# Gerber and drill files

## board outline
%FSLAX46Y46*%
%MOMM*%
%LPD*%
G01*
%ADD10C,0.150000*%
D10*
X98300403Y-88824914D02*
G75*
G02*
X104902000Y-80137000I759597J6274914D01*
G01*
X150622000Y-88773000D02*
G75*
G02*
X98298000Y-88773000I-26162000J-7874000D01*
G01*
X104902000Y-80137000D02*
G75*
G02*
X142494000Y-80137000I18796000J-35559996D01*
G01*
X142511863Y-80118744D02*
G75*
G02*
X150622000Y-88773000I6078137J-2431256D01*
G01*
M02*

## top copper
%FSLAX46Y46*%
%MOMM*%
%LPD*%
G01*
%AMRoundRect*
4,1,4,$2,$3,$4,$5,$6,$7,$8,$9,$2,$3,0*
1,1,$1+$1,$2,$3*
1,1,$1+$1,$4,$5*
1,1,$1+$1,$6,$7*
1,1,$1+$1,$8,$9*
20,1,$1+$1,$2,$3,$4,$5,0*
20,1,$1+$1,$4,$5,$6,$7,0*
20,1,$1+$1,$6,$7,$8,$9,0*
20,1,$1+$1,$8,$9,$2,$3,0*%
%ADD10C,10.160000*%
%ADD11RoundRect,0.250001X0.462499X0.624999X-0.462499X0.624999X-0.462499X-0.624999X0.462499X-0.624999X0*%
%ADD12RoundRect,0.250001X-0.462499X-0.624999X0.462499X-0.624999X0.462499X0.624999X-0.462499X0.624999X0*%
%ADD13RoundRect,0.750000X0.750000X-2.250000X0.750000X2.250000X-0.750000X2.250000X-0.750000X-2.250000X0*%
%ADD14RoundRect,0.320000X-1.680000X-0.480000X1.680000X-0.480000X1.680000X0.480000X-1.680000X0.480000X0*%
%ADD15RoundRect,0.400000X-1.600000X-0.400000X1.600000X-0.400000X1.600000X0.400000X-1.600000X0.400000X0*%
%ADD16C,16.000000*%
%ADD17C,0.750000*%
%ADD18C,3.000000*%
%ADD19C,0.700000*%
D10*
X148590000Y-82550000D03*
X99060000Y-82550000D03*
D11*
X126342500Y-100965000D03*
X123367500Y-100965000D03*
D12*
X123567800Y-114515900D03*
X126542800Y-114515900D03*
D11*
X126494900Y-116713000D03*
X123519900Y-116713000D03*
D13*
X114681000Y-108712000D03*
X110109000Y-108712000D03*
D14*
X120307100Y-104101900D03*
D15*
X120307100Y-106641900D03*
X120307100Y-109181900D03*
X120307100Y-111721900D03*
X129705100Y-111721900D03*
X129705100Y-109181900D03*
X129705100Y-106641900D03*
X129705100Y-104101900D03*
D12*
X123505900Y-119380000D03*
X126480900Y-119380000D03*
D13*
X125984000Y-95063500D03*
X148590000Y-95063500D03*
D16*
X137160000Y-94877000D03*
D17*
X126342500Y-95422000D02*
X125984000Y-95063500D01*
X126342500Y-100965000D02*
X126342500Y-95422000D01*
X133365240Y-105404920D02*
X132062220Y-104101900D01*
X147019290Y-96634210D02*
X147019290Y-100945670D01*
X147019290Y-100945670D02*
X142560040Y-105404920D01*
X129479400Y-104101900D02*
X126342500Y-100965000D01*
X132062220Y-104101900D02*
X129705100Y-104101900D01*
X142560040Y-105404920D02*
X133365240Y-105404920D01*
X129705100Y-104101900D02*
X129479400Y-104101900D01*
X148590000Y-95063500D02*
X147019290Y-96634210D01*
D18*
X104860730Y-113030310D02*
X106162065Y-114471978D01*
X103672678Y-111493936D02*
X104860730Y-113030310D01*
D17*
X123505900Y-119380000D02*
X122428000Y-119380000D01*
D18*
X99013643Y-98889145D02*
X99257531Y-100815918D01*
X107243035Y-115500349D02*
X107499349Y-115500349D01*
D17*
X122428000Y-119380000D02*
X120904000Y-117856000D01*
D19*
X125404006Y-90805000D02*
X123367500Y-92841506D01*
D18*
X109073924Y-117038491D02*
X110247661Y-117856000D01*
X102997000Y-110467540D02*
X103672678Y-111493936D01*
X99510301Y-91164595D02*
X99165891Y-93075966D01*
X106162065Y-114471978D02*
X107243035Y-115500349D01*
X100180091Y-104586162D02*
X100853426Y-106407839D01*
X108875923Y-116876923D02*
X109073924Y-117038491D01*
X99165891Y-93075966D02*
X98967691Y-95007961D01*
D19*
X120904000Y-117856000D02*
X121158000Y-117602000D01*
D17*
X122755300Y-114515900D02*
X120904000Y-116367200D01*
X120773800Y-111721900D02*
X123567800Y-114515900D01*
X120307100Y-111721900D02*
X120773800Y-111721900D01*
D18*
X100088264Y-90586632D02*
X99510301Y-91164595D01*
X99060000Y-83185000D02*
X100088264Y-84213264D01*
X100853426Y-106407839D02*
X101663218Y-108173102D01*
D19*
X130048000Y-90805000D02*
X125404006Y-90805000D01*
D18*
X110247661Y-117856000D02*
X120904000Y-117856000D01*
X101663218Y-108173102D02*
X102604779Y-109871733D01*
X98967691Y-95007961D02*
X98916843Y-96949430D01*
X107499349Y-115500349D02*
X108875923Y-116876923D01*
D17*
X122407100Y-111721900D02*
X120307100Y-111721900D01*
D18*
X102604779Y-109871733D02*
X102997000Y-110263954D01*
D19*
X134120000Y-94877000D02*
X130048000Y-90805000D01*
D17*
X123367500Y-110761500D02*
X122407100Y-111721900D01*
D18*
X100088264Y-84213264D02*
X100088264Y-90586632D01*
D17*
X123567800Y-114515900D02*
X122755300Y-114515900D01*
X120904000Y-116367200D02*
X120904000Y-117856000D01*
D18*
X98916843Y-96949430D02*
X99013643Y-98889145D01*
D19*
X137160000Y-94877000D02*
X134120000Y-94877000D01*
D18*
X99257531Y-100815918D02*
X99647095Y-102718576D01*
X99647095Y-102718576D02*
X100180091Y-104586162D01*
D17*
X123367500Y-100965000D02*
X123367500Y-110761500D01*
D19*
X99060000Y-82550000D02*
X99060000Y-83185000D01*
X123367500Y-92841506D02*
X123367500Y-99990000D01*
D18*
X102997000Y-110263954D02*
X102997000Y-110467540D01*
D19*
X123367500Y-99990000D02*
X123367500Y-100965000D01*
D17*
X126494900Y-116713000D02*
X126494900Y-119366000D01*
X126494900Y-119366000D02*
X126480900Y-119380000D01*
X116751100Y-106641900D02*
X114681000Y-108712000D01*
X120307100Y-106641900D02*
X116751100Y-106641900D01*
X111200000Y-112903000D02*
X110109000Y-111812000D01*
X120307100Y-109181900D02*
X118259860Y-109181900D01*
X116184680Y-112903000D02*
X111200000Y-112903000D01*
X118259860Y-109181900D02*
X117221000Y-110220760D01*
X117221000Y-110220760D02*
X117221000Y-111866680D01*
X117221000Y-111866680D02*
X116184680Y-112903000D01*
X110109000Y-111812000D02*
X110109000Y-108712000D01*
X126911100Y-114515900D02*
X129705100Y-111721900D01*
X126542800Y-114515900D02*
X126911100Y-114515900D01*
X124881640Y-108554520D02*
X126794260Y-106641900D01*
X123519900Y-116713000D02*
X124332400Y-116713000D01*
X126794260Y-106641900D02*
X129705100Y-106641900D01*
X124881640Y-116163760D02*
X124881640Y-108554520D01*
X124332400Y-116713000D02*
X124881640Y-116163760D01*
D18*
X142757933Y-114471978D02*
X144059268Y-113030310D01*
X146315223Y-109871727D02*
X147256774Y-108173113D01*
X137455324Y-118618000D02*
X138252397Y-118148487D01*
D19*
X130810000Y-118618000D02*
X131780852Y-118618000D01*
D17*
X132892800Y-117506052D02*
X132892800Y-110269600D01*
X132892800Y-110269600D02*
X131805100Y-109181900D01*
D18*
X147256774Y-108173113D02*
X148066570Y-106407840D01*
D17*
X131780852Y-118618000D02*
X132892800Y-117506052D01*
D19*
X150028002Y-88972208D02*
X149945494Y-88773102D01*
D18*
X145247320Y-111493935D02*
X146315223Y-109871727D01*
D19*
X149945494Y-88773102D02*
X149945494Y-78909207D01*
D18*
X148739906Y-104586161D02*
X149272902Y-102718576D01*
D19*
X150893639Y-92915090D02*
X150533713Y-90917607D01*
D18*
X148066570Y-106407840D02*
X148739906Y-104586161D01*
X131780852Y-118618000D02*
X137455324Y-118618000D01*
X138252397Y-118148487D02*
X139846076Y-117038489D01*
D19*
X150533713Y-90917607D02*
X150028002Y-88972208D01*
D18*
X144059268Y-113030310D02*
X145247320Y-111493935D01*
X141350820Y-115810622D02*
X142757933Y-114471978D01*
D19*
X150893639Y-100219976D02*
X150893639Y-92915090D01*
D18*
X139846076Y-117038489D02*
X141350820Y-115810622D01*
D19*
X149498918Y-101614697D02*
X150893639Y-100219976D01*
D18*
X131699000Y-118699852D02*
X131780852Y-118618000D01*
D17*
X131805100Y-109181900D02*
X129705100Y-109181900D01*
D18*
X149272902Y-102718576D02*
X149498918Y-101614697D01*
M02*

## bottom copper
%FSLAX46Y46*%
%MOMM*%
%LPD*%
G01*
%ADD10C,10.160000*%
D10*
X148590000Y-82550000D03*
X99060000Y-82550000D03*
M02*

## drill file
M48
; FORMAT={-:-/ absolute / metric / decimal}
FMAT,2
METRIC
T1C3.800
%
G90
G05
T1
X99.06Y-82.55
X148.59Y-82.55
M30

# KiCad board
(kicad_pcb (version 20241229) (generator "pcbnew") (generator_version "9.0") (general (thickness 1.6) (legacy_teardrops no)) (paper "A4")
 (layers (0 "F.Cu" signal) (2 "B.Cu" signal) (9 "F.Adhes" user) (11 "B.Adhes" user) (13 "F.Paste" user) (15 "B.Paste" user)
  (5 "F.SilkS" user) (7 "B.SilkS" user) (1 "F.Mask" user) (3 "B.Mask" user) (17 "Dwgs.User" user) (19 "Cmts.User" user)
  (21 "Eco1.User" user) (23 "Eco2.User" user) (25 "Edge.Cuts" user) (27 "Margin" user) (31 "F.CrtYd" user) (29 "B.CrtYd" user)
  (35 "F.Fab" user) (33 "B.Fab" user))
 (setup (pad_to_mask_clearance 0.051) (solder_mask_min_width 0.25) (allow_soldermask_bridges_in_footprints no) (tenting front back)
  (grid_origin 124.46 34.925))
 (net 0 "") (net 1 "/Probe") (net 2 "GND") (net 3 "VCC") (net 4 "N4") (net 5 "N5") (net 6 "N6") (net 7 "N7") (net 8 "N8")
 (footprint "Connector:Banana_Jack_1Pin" (layer "F.Cu") (at 148.59 82.55)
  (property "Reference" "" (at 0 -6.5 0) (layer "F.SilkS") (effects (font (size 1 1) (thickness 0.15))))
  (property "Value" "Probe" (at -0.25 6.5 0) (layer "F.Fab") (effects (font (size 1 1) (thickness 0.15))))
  (pad "1" thru_hole circle (at 0 0) (size 10.16 10.16) (drill 3.8) (layers "*.Cu" "*.Mask") (remove_unused_layers no) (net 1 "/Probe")))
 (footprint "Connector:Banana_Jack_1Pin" (layer "F.Cu") (at 99.06 82.55)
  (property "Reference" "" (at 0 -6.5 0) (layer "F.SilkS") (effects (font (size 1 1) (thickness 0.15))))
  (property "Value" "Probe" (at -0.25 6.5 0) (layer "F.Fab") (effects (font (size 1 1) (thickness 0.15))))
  (pad "1" thru_hole circle (at 0 0) (size 10.16 10.16) (drill 3.8) (layers "*.Cu" "*.Mask") (remove_unused_layers no) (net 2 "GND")))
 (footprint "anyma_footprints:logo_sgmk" (layer "F.Cu") (at 135.382 110.744)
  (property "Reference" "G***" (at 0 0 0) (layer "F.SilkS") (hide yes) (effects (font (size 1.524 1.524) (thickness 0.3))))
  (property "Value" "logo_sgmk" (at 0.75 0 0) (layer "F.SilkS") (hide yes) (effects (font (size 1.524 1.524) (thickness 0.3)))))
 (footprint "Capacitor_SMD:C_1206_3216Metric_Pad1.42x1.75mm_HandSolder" (layer "F.Cu") (at 124.855 100.965 180)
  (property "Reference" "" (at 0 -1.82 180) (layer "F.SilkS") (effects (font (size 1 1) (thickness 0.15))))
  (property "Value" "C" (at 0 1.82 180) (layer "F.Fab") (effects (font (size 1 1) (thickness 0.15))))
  (pad "1" smd roundrect (at -1.4875 0 180) (size 1.425 1.75) (layers "F.Cu" "F.Mask" "F.Paste") (roundrect_rratio 0.175439) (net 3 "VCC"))
  (pad "2" smd roundrect (at 1.4875 0 180) (size 1.425 1.75) (layers "F.Cu" "F.Mask" "F.Paste") (roundrect_rratio 0.175439) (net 2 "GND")))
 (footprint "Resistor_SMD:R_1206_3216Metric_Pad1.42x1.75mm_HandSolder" (layer "F.Cu") (at 125.0553 114.5159)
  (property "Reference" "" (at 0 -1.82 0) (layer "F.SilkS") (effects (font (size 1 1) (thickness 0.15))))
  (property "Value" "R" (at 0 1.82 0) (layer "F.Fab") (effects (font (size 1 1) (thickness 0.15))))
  (pad "1" smd roundrect (at -1.4875 0) (size 1.425 1.75) (layers "F.Cu" "F.Mask" "F.Paste") (roundrect_rratio 0.175439) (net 2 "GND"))
  (pad "2" smd roundrect (at 1.4875 0) (size 1.425 1.75) (layers "F.Cu" "F.Mask" "F.Paste") (roundrect_rratio 0.175439) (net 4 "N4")))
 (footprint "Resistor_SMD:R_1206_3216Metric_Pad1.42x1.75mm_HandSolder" (layer "F.Cu") (at 125.0074 116.713 180)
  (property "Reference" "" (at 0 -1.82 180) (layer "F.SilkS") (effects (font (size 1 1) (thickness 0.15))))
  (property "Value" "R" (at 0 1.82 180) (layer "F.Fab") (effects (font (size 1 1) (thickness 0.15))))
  (pad "1" smd roundrect (at -1.4875 0 180) (size 1.425 1.75) (layers "F.Cu" "F.Mask" "F.Paste") (roundrect_rratio 0.175439) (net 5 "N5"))
  (pad "2" smd roundrect (at 1.4875 0 180) (size 1.425 1.75) (layers "F.Cu" "F.Mask" "F.Paste") (roundrect_rratio 0.175439) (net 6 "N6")))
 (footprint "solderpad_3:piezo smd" (layer "F.Cu") (at 112.395 93.98 -90)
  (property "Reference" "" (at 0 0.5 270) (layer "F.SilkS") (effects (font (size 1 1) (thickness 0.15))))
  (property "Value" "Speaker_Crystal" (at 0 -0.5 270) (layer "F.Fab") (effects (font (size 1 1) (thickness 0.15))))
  (pad "1" smd roundrect (at 14.732 -2.286 90) (size 6 3) (layers "F.Cu" "F.Mask" "F.Paste") (roundrect_rratio 0.25) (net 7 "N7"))
  (pad "2" smd roundrect (at 14.732 2.286 90) (size 6 3) (layers "F.Cu" "F.Mask" "F.Paste") (roundrect_rratio 0.25) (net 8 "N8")))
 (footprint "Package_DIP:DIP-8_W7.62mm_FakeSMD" (layer "F.Cu") (at 121.1961 104.1019)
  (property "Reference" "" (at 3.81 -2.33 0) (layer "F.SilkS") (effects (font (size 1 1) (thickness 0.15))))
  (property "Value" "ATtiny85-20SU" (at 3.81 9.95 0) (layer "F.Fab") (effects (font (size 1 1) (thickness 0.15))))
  (pad "1" smd roundrect (at -0.889 0) (size 4 1.6) (layers "F.Cu" "F.Mask" "F.Paste") (roundrect_rratio 0.2))
  (pad "2" smd roundrect (at -0.889 2.54) (size 4 1.6) (layers "F.Cu" "F.Mask" "F.Paste") (roundrect_rratio 0.25) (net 7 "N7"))
  (pad "3" smd roundrect (at -0.889 5.08) (size 4 1.6) (layers "F.Cu" "F.Mask" "F.Paste") (roundrect_rratio 0.25) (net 8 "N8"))
  (pad "4" smd roundrect (at -0.889 7.62) (size 4 1.6) (layers "F.Cu" "F.Mask" "F.Paste") (roundrect_rratio 0.25) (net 2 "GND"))
  (pad "5" smd roundrect (at 8.509 7.62) (size 4 1.6) (layers "F.Cu" "F.Mask" "F.Paste") (roundrect_rratio 0.25) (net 4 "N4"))
  (pad "6" smd roundrect (at 8.509 5.08) (size 4 1.6) (layers "F.Cu" "F.Mask" "F.Paste") (roundrect_rratio 0.25) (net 1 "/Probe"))
  (pad "7" smd roundrect (at 8.509 2.54) (size 4 1.6) (layers "F.Cu" "F.Mask" "F.Paste") (roundrect_rratio 0.25) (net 6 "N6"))
  (pad "8" smd roundrect (at 8.509 0) (size 4 1.6) (layers "F.Cu" "F.Mask" "F.Paste") (roundrect_rratio 0.25) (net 3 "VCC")))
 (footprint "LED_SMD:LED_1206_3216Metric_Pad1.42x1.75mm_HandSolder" (layer "F.Cu") (at 124.9934 119.38)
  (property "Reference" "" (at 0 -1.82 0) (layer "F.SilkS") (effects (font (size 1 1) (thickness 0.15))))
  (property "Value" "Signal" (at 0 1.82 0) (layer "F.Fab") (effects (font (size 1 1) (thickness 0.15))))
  (pad "1" smd roundrect (at -1.4875 0) (size 1.425 1.75) (layers "F.Cu" "F.Mask" "F.Paste") (roundrect_rratio 0.175439) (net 2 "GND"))
  (pad "2" smd roundrect (at 1.4875 0) (size 1.425 1.75) (layers "F.Cu" "F.Mask" "F.Paste") (roundrect_rratio 0.175439) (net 5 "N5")))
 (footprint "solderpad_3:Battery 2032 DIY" (layer "F.Cu") (at 137.16 95.0635)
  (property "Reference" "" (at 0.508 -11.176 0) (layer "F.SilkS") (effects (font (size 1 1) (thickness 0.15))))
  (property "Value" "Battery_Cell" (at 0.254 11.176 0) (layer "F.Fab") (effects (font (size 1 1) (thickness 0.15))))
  (pad "1" smd roundrect (at -11.176 0 90) (size 6 3) (layers "F.Cu" "F.Mask" "F.Paste") (roundrect_rratio 0.25) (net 3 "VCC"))
  (pad "1" smd roundrect (at 11.43 0 90) (size 6 3) (layers "F.Cu" "F.Mask" "F.Paste") (roundrect_rratio 0.25) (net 3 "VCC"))
  (pad "2" smd circle (at 0 -0.1865) (size 16 16) (layers "F.Cu" "F.Mask" "F.Paste") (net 2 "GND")))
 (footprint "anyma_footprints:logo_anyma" (layer "B.Cu") (at 125.222 99.441 180)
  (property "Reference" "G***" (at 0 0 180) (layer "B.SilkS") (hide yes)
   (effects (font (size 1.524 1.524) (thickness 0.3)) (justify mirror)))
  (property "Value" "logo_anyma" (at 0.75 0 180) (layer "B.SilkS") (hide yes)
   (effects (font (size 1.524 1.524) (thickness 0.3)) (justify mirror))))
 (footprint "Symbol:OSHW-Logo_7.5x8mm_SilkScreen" (layer "B.Cu") (at 125.349 111.506 180)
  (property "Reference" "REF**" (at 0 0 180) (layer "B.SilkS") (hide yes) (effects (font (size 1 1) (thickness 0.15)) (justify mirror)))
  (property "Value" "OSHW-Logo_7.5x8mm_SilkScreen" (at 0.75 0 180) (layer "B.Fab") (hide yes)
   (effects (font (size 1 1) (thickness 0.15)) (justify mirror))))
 (gr_arc (start 98.300403 88.824914) (mid 94.02734 78.725884) (end 104.902 80.137) (stroke (width 0.15) (type solid)) (layer "Edge.Cuts"))
 (gr_arc (start 150.622 88.773) (mid 124.46 123.968239) (end 98.298 88.773) (stroke (width 0.15) (type solid)) (layer "Edge.Cuts"))
 (gr_arc (start 104.902 80.137) (mid 123.698 75.475075) (end 142.494 80.137) (stroke (width 0.15) (type solid)) (layer "Edge.Cuts"))
 (gr_arc (start 142.511863 80.118744) (mid 153.366698 78.073627) (end 150.622 88.773) (stroke (width 0.15) (type solid)) (layer "Edge.Cuts"))
 (segment (start 126.3425 95.422) (end 125.984 95.0635) (width 0.75) (layer "F.Cu") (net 3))
 (segment (start 126.3425 100.965) (end 126.3425 95.422) (width 0.75) (layer "F.Cu") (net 3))
 (segment (start 133.36524 105.40492) (end 132.06222 104.1019) (width 0.75) (layer "F.Cu") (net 3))
 (segment (start 147.01929 96.63421) (end 147.01929 100.94567) (width 0.75) (layer "F.Cu") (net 3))
 (segment (start 147.01929 100.94567) (end 142.56004 105.40492) (width 0.75) (layer "F.Cu") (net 3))
 (segment (start 129.4794 104.1019) (end 126.3425 100.965) (width 0.75) (layer "F.Cu") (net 3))
 (segment (start 132.06222 104.1019) (end 129.7051 104.1019) (width 0.75) (layer "F.Cu") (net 3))
 (segment (start 142.56004 105.40492) (end 133.36524 105.40492) (width 0.75) (layer "F.Cu") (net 3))
 (segment (start 129.7051 104.1019) (end 129.4794 104.1019) (width 0.75) (layer "F.Cu") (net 3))
 (segment (start 148.59 95.0635) (end 147.01929 96.63421) (width 0.75) (layer "F.Cu") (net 3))
 (segment (start 104.86073 113.03031) (end 106.162065 114.471978) (width 3) (layer "F.Cu") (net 2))
 (segment (start 103.672678 111.493936) (end 104.86073 113.03031) (width 3) (layer "F.Cu") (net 2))
 (segment (start 123.5059 119.38) (end 122.428 119.38) (width 0.75) (layer "F.Cu") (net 2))
 (segment (start 99.013643 98.889145) (end 99.257531 100.815918) (width 3) (layer "F.Cu") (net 2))
 (segment (start 107.243035 115.500349) (end 107.499349 115.500349) (width 3) (layer "F.Cu") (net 2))
 (segment (start 122.428 119.38) (end 120.904 117.856) (width 0.75) (layer "F.Cu") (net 2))
 (segment (start 125.404006 90.805) (end 123.3675 92.841506) (width 0.7) (layer "F.Cu") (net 2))
 (segment (start 109.073924 117.038491) (end 110.247661 117.856) (width 3) (layer "F.Cu") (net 2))
 (segment (start 102.997 110.46754) (end 103.672678 111.493936) (width 3) (layer "F.Cu") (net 2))
 (segment (start 99.510301 91.164595) (end 99.165891 93.075966) (width 3) (layer "F.Cu") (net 2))
 (segment (start 106.162065 114.471978) (end 107.243035 115.500349) (width 3) (layer "F.Cu") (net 2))
 (segment (start 100.180091 104.586162) (end 100.853426 106.407839) (width 3) (layer "F.Cu") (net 2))
 (segment (start 108.875923 116.876923) (end 109.073924 117.038491) (width 3) (layer "F.Cu") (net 2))
 (segment (start 99.165891 93.075966) (end 98.967691 95.007961) (width 3) (layer "F.Cu") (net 2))
 (segment (start 120.904 117.856) (end 121.158 117.602) (width 0.7) (layer "F.Cu") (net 2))
 (segment (start 122.7553 114.5159) (end 120.904 116.3672) (width 0.75) (layer "F.Cu") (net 2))
 (segment (start 120.7738 111.7219) (end 123.5678 114.5159) (width 0.75) (layer "F.Cu") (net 2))
 (segment (start 120.3071 111.7219) (end 120.7738 111.7219) (width 0.75) (layer "F.Cu") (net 2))
 (segment (start 100.088264 90.586632) (end 99.510301 91.164595) (width 3) (layer "F.Cu") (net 2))
 (segment (start 99.06 83.185) (end 100.088264 84.213264) (width 3) (layer "F.Cu") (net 2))
 (segment (start 100.853426 106.407839) (end 101.663218 108.173102) (width 3) (layer "F.Cu") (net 2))
 (segment (start 130.048 90.805) (end 125.404006 90.805) (width 0.7) (layer "F.Cu") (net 2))
 (segment (start 110.247661 117.856) (end 120.904 117.856) (width 3) (layer "F.Cu") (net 2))
 (segment (start 101.663218 108.173102) (end 102.604779 109.871733) (width 3) (layer "F.Cu") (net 2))
 (segment (start 98.967691 95.007961) (end 98.916843 96.94943) (width 3) (layer "F.Cu") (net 2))
 (segment (start 107.499349 115.500349) (end 108.875923 116.876923) (width 3) (layer "F.Cu") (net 2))
 (segment (start 122.4071 111.7219) (end 120.3071 111.7219) (width 0.75) (layer "F.Cu") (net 2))
 (segment (start 102.604779 109.871733) (end 102.997 110.263954) (width 3) (layer "F.Cu") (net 2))
 (segment (start 134.12 94.877) (end 130.048 90.805) (width 0.7) (layer "F.Cu") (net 2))
 (segment (start 123.3675 110.7615) (end 122.4071 111.7219) (width 0.75) (layer "F.Cu") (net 2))
 (segment (start 100.088264 84.213264) (end 100.088264 90.586632) (width 3) (layer "F.Cu") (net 2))
 (segment (start 123.5678 114.5159) (end 122.7553 114.5159) (width 0.75) (layer "F.Cu") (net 2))
 (segment (start 120.904 116.3672) (end 120.904 117.856) (width 0.75) (layer "F.Cu") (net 2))
 (segment (start 98.916843 96.94943) (end 99.013643 98.889145) (width 3) (layer "F.Cu") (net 2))
 (segment (start 137.16 94.877) (end 134.12 94.877) (width 0.7) (layer "F.Cu") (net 2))
 (segment (start 99.257531 100.815918) (end 99.647095 102.718576) (width 3) (layer "F.Cu") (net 2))
 (segment (start 99.647095 102.718576) (end 100.180091 104.586162) (width 3) (layer "F.Cu") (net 2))
 (segment (start 123.3675 100.965) (end 123.3675 110.7615) (width 0.75) (layer "F.Cu") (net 2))
 (segment (start 99.06 82.55) (end 99.06 83.185) (width 0.7) (layer "F.Cu") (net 2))
 (segment (start 123.3675 92.841506) (end 123.3675 99.99) (width 0.7) (layer "F.Cu") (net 2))
 (segment (start 102.997 110.263954) (end 102.997 110.46754) (width 3) (layer "F.Cu") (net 2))
 (segment (start 123.3675 99.99) (end 123.3675 100.965) (width 0.7) (layer "F.Cu") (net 2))
 (segment (start 126.4949 116.713) (end 126.4949 119.366) (width 0.75) (layer "F.Cu") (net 5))
 (segment (start 126.4949 119.366) (end 126.4809 119.38) (width 0.75) (layer "F.Cu") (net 5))
 (segment (start 116.7511 106.6419) (end 114.681 108.712) (width 0.75) (layer "F.Cu") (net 7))
 (segment (start 120.3071 106.6419) (end 116.7511 106.6419) (width 0.75) (layer "F.Cu") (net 7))
 (segment (start 111.2 112.903) (end 110.109 111.812) (width 0.75) (layer "F.Cu") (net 8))
 (segment (start 120.3071 109.1819) (end 118.25986 109.1819) (width 0.75) (layer "F.Cu") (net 8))
 (segment (start 116.18468 112.903) (end 111.2 112.903) (width 0.75) (layer "F.Cu") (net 8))
 (segment (start 118.25986 109.1819) (end 117.221 110.22076) (width 0.75) (layer "F.Cu") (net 8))
 (segment (start 117.221 110.22076) (end 117.221 111.86668) (width 0.75) (layer "F.Cu") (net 8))
 (segment (start 117.221 111.86668) (end 116.18468 112.903) (width 0.75) (layer "F.Cu") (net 8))
 (segment (start 110.109 111.812) (end 110.109 108.712) (width 0.75) (layer "F.Cu") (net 8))
 (segment (start 126.9111 114.5159) (end 129.7051 111.7219) (width 0.75) (layer "F.Cu") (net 4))
 (segment (start 126.5428 114.5159) (end 126.9111 114.5159) (width 0.75) (layer "F.Cu") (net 4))
 (segment (start 124.88164 108.55452) (end 126.79426 106.6419) (width 0.75) (layer "F.Cu") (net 6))
 (segment (start 123.5199 116.713) (end 124.3324 116.713) (width 0.75) (layer "F.Cu") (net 6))
 (segment (start 126.79426 106.6419) (end 129.7051 106.6419) (width 0.75) (layer "F.Cu") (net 6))
 (segment (start 124.88164 116.16376) (end 124.88164 108.55452) (width 0.75) (layer "F.Cu") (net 6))
 (segment (start 124.3324 116.713) (end 124.88164 116.16376) (width 0.75) (layer "F.Cu") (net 6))
 (segment (start 142.757933 114.471978) (end 144.059268 113.03031) (width 3) (layer "F.Cu") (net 1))
 (segment (start 146.315223 109.871727) (end 147.256774 108.173113) (width 3) (layer "F.Cu") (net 1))
 (segment (start 137.455324 118.618) (end 138.252397 118.148487) (width 3) (layer "F.Cu") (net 1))
 (segment (start 130.81 118.618) (end 131.780852 118.618) (width 0.7) (layer "F.Cu") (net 1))
 (segment (start 132.8928 117.506052) (end 132.8928 110.2696) (width 0.75) (layer "F.Cu") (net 1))
 (segment (start 132.8928 110.2696) (end 131.8051 109.1819) (width 0.75) (layer "F.Cu") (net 1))
 (segment (start 147.256774 108.173113) (end 148.06657 106.40784) (width 3) (layer "F.Cu") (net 1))
 (segment (start 131.780852 118.618) (end 132.8928 117.506052) (width 0.75) (layer "F.Cu") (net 1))
 (segment (start 150.028002 88.972208) (end 149.945494 88.773102) (width 0.7) (layer "F.Cu") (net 1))
 (segment (start 145.24732 111.493935) (end 146.315223 109.871727) (width 3) (layer "F.Cu") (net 1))
 (segment (start 149.945494 88.773102) (end 149.945494 78.909207) (width 0.7) (layer "F.Cu") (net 1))
 (segment (start 148.739906 104.586161) (end 149.272902 102.718576) (width 3) (layer "F.Cu") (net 1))
 (segment (start 150.893639 92.91509) (end 150.533713 90.917607) (width 0.7) (layer "F.Cu") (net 1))
 (segment (start 148.06657 106.40784) (end 148.739906 104.586161) (width 3) (layer "F.Cu") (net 1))
 (segment (start 131.780852 118.618) (end 137.455324 118.618) (width 3) (layer "F.Cu") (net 1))
 (segment (start 138.252397 118.148487) (end 139.846076 117.038489) (width 3) (layer "F.Cu") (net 1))
 (segment (start 150.533713 90.917607) (end 150.028002 88.972208) (width 0.7) (layer "F.Cu") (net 1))
 (segment (start 144.059268 113.03031) (end 145.24732 111.493935) (width 3) (layer "F.Cu") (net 1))
 (segment (start 141.35082 115.810622) (end 142.757933 114.471978) (width 3) (layer "F.Cu") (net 1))
 (segment (start 150.893639 100.219976) (end 150.893639 92.91509) (width 0.7) (layer "F.Cu") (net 1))
 (segment (start 139.846076 117.038489) (end 141.35082 115.810622) (width 3) (layer "F.Cu") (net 1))
 (segment (start 149.498918 101.614697) (end 150.893639 100.219976) (width 0.7) (layer "F.Cu") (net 1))
 (segment (start 131.699 118.699852) (end 131.780852 118.618) (width 3) (layer "F.Cu") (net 1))
 (segment (start 131.8051 109.1819) (end 129.7051 109.1819) (width 0.75) (layer "F.Cu") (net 1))
 (segment (start 149.272902 102.718576) (end 149.498918 101.614697) (width 3) (layer "F.Cu") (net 1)))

